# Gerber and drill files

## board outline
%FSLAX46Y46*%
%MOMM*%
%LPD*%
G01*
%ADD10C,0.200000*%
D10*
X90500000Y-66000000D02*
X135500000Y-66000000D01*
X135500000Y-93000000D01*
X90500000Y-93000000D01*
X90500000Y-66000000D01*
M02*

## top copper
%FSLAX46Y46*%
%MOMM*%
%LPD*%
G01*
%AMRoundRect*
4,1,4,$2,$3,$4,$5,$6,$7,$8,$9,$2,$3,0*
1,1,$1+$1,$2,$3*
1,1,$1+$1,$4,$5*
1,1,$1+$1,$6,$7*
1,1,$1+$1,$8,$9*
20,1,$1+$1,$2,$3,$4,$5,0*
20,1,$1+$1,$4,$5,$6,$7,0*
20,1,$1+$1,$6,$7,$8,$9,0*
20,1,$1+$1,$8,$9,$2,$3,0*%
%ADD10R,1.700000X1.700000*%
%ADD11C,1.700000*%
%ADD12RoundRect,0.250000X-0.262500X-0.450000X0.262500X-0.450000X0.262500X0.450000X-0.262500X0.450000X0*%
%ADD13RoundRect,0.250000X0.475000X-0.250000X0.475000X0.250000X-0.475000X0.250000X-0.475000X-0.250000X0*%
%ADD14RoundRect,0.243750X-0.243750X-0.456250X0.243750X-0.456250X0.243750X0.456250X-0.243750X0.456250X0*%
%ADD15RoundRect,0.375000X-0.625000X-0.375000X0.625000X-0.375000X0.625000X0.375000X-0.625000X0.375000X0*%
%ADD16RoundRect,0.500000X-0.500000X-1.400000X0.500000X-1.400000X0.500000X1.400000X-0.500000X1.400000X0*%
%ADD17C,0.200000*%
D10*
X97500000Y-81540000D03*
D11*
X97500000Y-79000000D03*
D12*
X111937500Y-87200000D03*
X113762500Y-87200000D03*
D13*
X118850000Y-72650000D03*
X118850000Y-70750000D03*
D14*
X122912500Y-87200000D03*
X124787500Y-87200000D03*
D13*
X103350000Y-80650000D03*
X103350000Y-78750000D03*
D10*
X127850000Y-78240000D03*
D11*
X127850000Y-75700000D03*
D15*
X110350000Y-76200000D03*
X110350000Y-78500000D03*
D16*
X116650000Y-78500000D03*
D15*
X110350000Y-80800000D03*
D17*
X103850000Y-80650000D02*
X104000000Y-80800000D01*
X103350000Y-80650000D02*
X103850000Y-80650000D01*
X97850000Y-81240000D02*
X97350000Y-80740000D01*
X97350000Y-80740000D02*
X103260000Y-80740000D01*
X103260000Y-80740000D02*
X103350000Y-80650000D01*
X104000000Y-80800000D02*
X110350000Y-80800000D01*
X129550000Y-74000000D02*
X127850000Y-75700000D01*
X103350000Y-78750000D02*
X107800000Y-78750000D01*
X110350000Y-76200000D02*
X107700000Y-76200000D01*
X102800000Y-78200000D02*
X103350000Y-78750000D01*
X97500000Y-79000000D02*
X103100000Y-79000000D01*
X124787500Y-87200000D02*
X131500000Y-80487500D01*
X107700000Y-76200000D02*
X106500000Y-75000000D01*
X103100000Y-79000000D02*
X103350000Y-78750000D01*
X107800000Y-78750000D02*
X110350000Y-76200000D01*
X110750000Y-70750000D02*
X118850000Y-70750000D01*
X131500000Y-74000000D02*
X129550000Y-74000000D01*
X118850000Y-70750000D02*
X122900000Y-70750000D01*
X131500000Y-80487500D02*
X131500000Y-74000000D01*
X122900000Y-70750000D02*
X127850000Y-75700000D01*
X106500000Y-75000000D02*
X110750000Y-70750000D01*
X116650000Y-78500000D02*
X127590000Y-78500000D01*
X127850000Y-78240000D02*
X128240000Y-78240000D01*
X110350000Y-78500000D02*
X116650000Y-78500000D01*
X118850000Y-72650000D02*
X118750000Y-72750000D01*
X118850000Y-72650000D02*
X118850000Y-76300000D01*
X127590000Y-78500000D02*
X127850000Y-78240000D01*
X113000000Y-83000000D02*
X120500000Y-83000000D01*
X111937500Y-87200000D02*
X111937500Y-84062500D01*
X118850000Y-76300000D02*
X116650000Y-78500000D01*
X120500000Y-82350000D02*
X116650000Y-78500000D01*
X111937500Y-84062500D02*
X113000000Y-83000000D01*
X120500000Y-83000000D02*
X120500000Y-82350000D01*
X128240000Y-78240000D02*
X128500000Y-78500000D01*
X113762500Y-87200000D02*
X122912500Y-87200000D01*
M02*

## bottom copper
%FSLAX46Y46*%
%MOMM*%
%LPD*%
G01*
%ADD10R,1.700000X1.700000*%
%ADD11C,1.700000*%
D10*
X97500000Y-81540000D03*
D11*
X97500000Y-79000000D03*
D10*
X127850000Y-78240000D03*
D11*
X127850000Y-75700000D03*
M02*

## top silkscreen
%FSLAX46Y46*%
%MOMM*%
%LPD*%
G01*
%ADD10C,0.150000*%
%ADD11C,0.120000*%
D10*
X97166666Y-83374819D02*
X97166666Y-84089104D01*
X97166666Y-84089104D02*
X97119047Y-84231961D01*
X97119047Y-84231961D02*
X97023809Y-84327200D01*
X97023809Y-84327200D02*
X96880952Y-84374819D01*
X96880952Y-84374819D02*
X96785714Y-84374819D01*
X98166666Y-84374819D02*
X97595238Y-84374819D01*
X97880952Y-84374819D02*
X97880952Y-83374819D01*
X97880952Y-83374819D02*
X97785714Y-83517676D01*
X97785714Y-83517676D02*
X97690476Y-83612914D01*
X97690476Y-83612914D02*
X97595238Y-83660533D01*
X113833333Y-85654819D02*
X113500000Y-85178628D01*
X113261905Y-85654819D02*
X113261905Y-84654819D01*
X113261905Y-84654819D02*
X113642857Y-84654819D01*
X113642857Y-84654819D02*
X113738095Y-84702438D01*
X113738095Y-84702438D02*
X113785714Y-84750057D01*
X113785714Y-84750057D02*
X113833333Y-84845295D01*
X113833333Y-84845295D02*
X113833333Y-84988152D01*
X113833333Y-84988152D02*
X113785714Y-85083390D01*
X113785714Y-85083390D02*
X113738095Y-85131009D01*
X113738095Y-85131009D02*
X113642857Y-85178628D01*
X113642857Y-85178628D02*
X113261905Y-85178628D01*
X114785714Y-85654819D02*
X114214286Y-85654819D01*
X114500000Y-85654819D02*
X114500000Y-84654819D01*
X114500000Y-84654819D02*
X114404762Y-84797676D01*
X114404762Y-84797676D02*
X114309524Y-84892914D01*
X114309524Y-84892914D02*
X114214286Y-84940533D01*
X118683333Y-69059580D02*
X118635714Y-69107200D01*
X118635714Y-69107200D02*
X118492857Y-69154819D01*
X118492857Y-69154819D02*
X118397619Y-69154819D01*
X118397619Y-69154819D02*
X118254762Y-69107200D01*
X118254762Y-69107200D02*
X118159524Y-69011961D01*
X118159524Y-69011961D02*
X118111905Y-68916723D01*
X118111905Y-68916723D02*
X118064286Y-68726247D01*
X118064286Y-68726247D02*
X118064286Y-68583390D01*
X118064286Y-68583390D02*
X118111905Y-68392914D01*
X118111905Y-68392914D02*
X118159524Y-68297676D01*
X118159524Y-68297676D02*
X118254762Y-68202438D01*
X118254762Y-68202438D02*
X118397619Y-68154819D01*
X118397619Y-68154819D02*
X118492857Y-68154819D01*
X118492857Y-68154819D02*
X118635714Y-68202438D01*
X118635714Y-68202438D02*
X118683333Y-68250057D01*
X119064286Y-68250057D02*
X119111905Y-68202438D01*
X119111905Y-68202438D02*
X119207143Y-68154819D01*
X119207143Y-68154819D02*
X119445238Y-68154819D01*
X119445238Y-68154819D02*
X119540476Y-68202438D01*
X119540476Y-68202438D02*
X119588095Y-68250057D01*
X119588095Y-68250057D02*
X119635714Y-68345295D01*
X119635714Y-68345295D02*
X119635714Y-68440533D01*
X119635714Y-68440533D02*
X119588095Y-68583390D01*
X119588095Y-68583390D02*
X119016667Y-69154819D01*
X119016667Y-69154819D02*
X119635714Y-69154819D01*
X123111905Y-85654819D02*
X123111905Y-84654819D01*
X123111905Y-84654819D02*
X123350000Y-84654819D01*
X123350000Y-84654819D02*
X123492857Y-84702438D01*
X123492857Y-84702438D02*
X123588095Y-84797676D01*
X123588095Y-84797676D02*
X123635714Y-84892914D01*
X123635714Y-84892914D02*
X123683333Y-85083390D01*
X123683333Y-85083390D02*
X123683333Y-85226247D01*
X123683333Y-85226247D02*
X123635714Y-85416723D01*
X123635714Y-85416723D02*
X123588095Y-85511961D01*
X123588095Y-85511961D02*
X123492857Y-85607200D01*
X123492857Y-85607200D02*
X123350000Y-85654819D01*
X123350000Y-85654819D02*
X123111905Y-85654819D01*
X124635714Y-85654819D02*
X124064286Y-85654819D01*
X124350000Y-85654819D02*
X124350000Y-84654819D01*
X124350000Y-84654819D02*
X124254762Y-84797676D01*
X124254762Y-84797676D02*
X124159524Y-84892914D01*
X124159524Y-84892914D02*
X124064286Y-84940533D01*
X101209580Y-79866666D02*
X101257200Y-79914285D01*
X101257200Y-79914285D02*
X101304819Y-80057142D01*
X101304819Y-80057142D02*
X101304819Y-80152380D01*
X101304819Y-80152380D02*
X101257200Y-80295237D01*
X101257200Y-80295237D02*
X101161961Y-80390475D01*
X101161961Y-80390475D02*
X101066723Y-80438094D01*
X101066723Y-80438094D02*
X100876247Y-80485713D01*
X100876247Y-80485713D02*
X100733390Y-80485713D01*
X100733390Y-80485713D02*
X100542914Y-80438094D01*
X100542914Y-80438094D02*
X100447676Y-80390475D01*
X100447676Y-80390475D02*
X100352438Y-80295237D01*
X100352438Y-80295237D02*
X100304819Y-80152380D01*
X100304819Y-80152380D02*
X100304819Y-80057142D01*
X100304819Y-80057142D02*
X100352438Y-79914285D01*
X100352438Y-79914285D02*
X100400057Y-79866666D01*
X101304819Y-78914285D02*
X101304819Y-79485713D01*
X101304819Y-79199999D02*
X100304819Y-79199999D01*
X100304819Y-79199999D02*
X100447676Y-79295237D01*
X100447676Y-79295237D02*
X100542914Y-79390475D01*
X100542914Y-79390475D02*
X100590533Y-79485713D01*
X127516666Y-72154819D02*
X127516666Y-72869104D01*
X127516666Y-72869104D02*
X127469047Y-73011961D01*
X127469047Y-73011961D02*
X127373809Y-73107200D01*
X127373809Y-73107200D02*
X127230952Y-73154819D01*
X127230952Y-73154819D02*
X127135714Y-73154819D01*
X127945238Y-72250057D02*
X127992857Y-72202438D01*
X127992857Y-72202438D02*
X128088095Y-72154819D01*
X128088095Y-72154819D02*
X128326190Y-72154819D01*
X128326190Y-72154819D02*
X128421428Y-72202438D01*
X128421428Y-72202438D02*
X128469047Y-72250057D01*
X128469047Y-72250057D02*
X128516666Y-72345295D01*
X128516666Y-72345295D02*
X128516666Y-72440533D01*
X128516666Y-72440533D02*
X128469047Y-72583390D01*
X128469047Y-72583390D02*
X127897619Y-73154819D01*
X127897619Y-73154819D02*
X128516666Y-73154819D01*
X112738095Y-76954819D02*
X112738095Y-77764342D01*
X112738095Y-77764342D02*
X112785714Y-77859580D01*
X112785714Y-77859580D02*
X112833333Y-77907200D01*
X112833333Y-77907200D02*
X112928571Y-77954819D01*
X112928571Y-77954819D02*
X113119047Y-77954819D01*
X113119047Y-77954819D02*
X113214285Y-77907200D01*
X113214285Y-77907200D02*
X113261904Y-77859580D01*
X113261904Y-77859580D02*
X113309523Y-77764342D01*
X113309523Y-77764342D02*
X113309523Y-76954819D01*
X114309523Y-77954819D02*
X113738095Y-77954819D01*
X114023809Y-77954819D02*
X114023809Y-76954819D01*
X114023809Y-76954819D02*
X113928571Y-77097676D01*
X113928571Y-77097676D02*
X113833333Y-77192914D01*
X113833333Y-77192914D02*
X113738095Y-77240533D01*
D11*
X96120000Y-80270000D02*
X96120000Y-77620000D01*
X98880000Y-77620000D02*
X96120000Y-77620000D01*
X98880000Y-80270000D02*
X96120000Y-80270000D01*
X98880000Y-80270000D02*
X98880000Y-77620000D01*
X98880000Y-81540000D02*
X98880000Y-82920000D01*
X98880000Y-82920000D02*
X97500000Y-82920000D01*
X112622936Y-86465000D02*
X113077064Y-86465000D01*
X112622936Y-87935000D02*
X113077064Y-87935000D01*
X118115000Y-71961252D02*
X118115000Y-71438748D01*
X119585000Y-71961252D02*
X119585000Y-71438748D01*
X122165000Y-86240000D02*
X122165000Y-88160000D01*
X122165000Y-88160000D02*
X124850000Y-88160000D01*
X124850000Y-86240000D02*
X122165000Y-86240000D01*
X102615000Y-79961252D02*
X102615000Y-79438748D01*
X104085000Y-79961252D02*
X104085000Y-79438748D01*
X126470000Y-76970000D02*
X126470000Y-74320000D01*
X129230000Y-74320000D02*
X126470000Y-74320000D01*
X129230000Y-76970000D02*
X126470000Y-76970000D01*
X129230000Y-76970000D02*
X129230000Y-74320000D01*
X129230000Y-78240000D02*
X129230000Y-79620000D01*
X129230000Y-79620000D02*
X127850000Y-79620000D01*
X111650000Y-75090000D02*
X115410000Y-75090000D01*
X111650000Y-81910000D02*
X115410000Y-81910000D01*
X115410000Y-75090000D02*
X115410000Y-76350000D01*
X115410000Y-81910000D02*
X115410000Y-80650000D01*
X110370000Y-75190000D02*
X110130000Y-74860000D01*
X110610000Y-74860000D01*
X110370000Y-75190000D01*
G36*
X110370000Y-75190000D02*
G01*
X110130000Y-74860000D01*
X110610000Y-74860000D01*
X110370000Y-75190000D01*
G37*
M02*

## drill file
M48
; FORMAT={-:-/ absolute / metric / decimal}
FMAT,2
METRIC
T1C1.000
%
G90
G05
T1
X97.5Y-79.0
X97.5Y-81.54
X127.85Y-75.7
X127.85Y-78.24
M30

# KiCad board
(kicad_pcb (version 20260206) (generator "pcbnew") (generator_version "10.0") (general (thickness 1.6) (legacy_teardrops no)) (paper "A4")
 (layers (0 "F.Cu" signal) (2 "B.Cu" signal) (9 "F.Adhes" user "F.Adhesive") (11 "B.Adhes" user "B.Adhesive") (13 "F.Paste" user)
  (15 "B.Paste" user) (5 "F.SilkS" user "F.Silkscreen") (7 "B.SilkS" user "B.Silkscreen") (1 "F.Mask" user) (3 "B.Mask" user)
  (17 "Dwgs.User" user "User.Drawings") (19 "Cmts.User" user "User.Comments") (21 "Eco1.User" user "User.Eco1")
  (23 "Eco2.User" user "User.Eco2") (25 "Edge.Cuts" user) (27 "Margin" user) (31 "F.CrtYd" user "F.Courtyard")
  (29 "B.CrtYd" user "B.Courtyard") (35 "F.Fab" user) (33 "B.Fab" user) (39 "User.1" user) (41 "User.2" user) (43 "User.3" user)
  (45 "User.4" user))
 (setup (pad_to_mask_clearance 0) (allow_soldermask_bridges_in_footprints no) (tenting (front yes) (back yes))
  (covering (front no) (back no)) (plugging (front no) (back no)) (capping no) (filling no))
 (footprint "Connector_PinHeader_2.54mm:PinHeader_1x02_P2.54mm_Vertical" (layer "F.Cu") (at 97.5 81.54 180)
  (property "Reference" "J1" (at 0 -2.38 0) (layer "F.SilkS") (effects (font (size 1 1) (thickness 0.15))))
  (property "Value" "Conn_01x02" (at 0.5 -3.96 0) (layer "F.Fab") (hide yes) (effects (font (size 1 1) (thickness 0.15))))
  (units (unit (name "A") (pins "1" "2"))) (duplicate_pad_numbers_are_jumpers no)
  (fp_line (start 1.38 1.27) (end 1.38 3.92) (stroke (width 0.12) (type solid)) (layer "F.SilkS"))
  (fp_line (start -1.38 3.92) (end 1.38 3.92) (stroke (width 0.12) (type solid)) (layer "F.SilkS"))
  (fp_line (start -1.38 1.27) (end 1.38 1.27) (stroke (width 0.12) (type solid)) (layer "F.SilkS"))
  (fp_line (start -1.38 1.27) (end -1.38 3.92) (stroke (width 0.12) (type solid)) (layer "F.SilkS"))
  (fp_line (start -1.38 0) (end -1.38 -1.38) (stroke (width 0.12) (type solid)) (layer "F.SilkS"))
  (fp_line (start -1.38 -1.38) (end 0 -1.38) (stroke (width 0.12) (type solid)) (layer "F.SilkS"))
  (pad "1" thru_hole rect (at 0 0 180) (size 1.7 1.7) (drill 1) (layers "*.Cu" "*.Mask") (remove_unused_layers no) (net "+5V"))
  (pad "2" thru_hole circle (at 0 2.54 180) (size 1.7 1.7) (drill 1) (layers "*.Cu" "*.Mask") (remove_unused_layers no) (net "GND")))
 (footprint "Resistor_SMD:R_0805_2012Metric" (layer "F.Cu") (at 112.85 87.2)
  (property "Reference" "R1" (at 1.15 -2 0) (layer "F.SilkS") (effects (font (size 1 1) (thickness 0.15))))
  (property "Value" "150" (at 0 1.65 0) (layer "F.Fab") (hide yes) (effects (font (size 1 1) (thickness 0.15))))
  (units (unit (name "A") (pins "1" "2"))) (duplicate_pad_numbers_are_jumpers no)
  (fp_line (start -0.227064 -0.735) (end 0.227064 -0.735) (stroke (width 0.12) (type solid)) (layer "F.SilkS"))
  (fp_line (start -0.227064 0.735) (end 0.227064 0.735) (stroke (width 0.12) (type solid)) (layer "F.SilkS"))
  (pad "1" smd roundrect (at -0.9125 0) (size 1.025 1.4) (layers "F.Cu" "F.Mask" "F.Paste") (roundrect_rratio 0.243902) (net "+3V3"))
  (pad "2" smd roundrect (at 0.9125 0) (size 1.025 1.4) (layers "F.Cu" "F.Mask" "F.Paste") (roundrect_rratio 0.243902) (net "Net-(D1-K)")))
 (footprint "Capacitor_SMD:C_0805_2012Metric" (layer "F.Cu") (at 118.85 71.7 90)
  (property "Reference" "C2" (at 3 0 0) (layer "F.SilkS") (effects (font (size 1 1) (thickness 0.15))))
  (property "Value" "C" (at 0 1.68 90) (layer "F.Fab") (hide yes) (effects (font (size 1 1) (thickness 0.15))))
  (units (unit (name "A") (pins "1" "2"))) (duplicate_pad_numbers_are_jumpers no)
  (fp_line (start -0.261252 -0.735) (end 0.261252 -0.735) (stroke (width 0.12) (type solid)) (layer "F.SilkS"))
  (fp_line (start -0.261252 0.735) (end 0.261252 0.735) (stroke (width 0.12) (type solid)) (layer "F.SilkS"))
  (pad "1" smd roundrect (at -0.95 0 90) (size 1 1.45) (layers "F.Cu" "F.Mask" "F.Paste") (roundrect_rratio 0.25) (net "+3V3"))
  (pad "2" smd roundrect (at 0.95 0 90) (size 1 1.45) (layers "F.Cu" "F.Mask" "F.Paste") (roundrect_rratio 0.25) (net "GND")))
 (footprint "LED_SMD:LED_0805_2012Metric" (layer "F.Cu") (at 123.85 87.2)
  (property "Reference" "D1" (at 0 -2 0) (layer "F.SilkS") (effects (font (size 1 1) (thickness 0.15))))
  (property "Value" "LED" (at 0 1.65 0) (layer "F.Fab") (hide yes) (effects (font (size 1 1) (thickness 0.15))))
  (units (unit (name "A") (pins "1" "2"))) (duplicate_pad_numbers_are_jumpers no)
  (fp_line (start -1.685 -0.96) (end -1.685 0.96) (stroke (width 0.12) (type solid)) (layer "F.SilkS"))
  (fp_line (start -1.685 0.96) (end 1 0.96) (stroke (width 0.12) (type solid)) (layer "F.SilkS"))
  (fp_line (start 1 -0.96) (end -1.685 -0.96) (stroke (width 0.12) (type solid)) (layer "F.SilkS"))
  (pad "1" smd roundrect (at -0.9375 0) (size 0.975 1.4) (layers "F.Cu" "F.Mask" "F.Paste") (roundrect_rratio 0.25) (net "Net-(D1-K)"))
  (pad "2" smd roundrect (at 0.9375 0) (size 0.975 1.4) (layers "F.Cu" "F.Mask" "F.Paste") (roundrect_rratio 0.25) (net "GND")))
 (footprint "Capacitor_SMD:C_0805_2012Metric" (layer "F.Cu") (at 103.35 79.7 90)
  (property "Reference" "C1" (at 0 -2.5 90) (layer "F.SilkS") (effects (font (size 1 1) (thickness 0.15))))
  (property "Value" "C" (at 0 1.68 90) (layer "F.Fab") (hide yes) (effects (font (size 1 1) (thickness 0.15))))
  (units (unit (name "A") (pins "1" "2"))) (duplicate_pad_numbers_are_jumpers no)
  (fp_line (start -0.261252 -0.735) (end 0.261252 -0.735) (stroke (width 0.12) (type solid)) (layer "F.SilkS"))
  (fp_line (start -0.261252 0.735) (end 0.261252 0.735) (stroke (width 0.12) (type solid)) (layer "F.SilkS"))
  (pad "1" smd roundrect (at -0.95 0 90) (size 1 1.45) (layers "F.Cu" "F.Mask" "F.Paste") (roundrect_rratio 0.25) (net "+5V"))
  (pad "2" smd roundrect (at 0.95 0 90) (size 1 1.45) (layers "F.Cu" "F.Mask" "F.Paste") (roundrect_rratio 0.25) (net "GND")))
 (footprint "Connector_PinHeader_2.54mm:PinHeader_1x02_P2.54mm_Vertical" (layer "F.Cu") (at 127.85 78.24 180)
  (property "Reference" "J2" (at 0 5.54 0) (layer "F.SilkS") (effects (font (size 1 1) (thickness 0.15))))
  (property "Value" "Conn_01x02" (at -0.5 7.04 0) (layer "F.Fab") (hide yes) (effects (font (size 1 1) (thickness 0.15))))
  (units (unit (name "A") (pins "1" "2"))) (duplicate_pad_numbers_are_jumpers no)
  (fp_line (start 1.38 1.27) (end 1.38 3.92) (stroke (width 0.12) (type solid)) (layer "F.SilkS"))
  (fp_line (start -1.38 3.92) (end 1.38 3.92) (stroke (width 0.12) (type solid)) (layer "F.SilkS"))
  (fp_line (start -1.38 1.27) (end 1.38 1.27) (stroke (width 0.12) (type solid)) (layer "F.SilkS"))
  (fp_line (start -1.38 1.27) (end -1.38 3.92) (stroke (width 0.12) (type solid)) (layer "F.SilkS"))
  (fp_line (start -1.38 0) (end -1.38 -1.38) (stroke (width 0.12) (type solid)) (layer "F.SilkS"))
  (fp_line (start -1.38 -1.38) (end 0 -1.38) (stroke (width 0.12) (type solid)) (layer "F.SilkS"))
  (pad "1" thru_hole rect (at 0 0 180) (size 1.7 1.7) (drill 1) (layers "*.Cu" "*.Mask") (remove_unused_layers no) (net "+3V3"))
  (pad "2" thru_hole circle (at 0 2.54 180) (size 1.7 1.7) (drill 1) (layers "*.Cu" "*.Mask") (remove_unused_layers no) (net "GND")))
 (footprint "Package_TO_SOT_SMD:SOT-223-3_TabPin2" (layer "F.Cu") (at 113.5 78.5)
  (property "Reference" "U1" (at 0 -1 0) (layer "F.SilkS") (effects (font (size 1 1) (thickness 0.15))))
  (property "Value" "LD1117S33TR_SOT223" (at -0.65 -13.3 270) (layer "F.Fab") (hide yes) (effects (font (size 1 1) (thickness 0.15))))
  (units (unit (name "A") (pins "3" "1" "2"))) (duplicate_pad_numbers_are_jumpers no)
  (fp_line (start -1.85 -3.41) (end 1.91 -3.41) (stroke (width 0.12) (type solid)) (layer "F.SilkS"))
  (fp_line (start -1.85 3.41) (end 1.91 3.41) (stroke (width 0.12) (type solid)) (layer "F.SilkS"))
  (fp_line (start 1.91 -3.41) (end 1.91 -2.15) (stroke (width 0.12) (type solid)) (layer "F.SilkS"))
  (fp_line (start 1.91 3.41) (end 1.91 2.15) (stroke (width 0.12) (type solid)) (layer "F.SilkS"))
  (fp_poly
   (pts (xy -3.13 -3.31) (xy -3.37 -3.64) (xy -2.89 -3.64) (xy -3.13 -3.31)) (stroke (width 0.12) (type solid)) (fill yes) (layer "F.SilkS"))
  (pad "1" smd roundrect (at -3.15 -2.3) (size 2 1.5) (layers "F.Cu" "F.Mask" "F.Paste") (roundrect_rratio 0.25) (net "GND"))
  (pad "2" smd roundrect (at -3.15 0) (size 2 1.5) (layers "F.Cu" "F.Mask" "F.Paste") (roundrect_rratio 0.25) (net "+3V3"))
  (pad "2" smd roundrect (at 3.15 0) (size 2 3.8) (layers "F.Cu" "F.Mask" "F.Paste") (roundrect_rratio 0.25) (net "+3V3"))
  (pad "3" smd roundrect (at -3.15 2.3) (size 2 1.5) (layers "F.Cu" "F.Mask" "F.Paste") (roundrect_rratio 0.25) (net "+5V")))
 (gr_rect (start 90.5 66) (end 135.5 93) (stroke (width 0.2) (type solid)) (fill no) (layer "Edge.Cuts"))
 (segment (start 103.85 80.65) (end 104 80.8) (width 0.2) (layer "F.Cu") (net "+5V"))
 (segment (start 103.35 80.65) (end 103.85 80.65) (width 0.2) (layer "F.Cu") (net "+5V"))
 (segment (start 97.85 81.24) (end 97.35 80.74) (width 0.2) (layer "F.Cu") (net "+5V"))
 (segment (start 97.35 80.74) (end 103.26 80.74) (width 0.2) (layer "F.Cu") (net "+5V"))
 (segment (start 103.26 80.74) (end 103.35 80.65) (width 0.2) (layer "F.Cu") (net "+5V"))
 (segment (start 104 80.8) (end 110.35 80.8) (width 0.2) (layer "F.Cu") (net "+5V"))
 (segment (start 129.55 74) (end 127.85 75.7) (width 0.2) (layer "F.Cu") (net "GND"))
 (segment (start 103.35 78.75) (end 107.8 78.75) (width 0.2) (layer "F.Cu") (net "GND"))
 (segment (start 110.35 76.2) (end 107.7 76.2) (width 0.2) (layer "F.Cu") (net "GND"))
 (segment (start 102.8 78.2) (end 103.35 78.75) (width 0.2) (layer "F.Cu") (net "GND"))
 (segment (start 97.5 79) (end 103.1 79) (width 0.2) (layer "F.Cu") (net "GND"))
 (segment (start 124.7875 87.2) (end 131.5 80.4875) (width 0.2) (layer "F.Cu") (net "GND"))
 (segment (start 107.7 76.2) (end 106.5 75) (width 0.2) (layer "F.Cu") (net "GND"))
 (segment (start 103.1 79) (end 103.35 78.75) (width 0.2) (layer "F.Cu") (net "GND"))
 (segment (start 107.8 78.75) (end 110.35 76.2) (width 0.2) (layer "F.Cu") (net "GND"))
 (segment (start 110.75 70.75) (end 118.85 70.75) (width 0.2) (layer "F.Cu") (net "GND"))
 (segment (start 131.5 74) (end 129.55 74) (width 0.2) (layer "F.Cu") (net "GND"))
 (segment (start 118.85 70.75) (end 122.9 70.75) (width 0.2) (layer "F.Cu") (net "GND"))
 (segment (start 131.5 80.4875) (end 131.5 74) (width 0.2) (layer "F.Cu") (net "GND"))
 (segment (start 122.9 70.75) (end 127.85 75.7) (width 0.2) (layer "F.Cu") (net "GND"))
 (segment (start 106.5 75) (end 110.75 70.75) (width 0.2) (layer "F.Cu") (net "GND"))
 (segment (start 116.65 78.5) (end 127.59 78.5) (width 0.2) (layer "F.Cu") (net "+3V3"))
 (segment (start 127.85 78.24) (end 128.24 78.24) (width 0.2) (layer "F.Cu") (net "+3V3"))
 (segment (start 110.35 78.5) (end 116.65 78.5) (width 0.2) (layer "F.Cu") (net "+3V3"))
 (segment (start 118.85 72.65) (end 118.75 72.75) (width 0.2) (layer "F.Cu") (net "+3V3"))
 (segment (start 118.85 72.65) (end 118.85 76.3) (width 0.2) (layer "F.Cu") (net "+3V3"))
 (segment (start 127.59 78.5) (end 127.85 78.24) (width 0.2) (layer "F.Cu") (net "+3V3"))
 (segment (start 113 83) (end 120.5 83) (width 0.2) (layer "F.Cu") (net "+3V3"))
 (segment (start 111.9375 87.2) (end 111.9375 84.0625) (width 0.2) (layer "F.Cu") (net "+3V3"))
 (segment (start 118.85 76.3) (end 116.65 78.5) (width 0.2) (layer "F.Cu") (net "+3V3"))
 (segment (start 120.5 82.35) (end 116.65 78.5) (width 0.2) (layer "F.Cu") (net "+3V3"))
 (segment (start 111.9375 84.0625) (end 113 83) (width 0.2) (layer "F.Cu") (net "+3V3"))
 (segment (start 120.5 83) (end 120.5 82.35) (width 0.2) (layer "F.Cu") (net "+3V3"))
 (segment (start 128.24 78.24) (end 128.5 78.5) (width 0.2) (layer "F.Cu") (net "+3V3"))
 (segment (start 113.7625 87.2) (end 122.9125 87.2) (width 0.2) (layer "F.Cu") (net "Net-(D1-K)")))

